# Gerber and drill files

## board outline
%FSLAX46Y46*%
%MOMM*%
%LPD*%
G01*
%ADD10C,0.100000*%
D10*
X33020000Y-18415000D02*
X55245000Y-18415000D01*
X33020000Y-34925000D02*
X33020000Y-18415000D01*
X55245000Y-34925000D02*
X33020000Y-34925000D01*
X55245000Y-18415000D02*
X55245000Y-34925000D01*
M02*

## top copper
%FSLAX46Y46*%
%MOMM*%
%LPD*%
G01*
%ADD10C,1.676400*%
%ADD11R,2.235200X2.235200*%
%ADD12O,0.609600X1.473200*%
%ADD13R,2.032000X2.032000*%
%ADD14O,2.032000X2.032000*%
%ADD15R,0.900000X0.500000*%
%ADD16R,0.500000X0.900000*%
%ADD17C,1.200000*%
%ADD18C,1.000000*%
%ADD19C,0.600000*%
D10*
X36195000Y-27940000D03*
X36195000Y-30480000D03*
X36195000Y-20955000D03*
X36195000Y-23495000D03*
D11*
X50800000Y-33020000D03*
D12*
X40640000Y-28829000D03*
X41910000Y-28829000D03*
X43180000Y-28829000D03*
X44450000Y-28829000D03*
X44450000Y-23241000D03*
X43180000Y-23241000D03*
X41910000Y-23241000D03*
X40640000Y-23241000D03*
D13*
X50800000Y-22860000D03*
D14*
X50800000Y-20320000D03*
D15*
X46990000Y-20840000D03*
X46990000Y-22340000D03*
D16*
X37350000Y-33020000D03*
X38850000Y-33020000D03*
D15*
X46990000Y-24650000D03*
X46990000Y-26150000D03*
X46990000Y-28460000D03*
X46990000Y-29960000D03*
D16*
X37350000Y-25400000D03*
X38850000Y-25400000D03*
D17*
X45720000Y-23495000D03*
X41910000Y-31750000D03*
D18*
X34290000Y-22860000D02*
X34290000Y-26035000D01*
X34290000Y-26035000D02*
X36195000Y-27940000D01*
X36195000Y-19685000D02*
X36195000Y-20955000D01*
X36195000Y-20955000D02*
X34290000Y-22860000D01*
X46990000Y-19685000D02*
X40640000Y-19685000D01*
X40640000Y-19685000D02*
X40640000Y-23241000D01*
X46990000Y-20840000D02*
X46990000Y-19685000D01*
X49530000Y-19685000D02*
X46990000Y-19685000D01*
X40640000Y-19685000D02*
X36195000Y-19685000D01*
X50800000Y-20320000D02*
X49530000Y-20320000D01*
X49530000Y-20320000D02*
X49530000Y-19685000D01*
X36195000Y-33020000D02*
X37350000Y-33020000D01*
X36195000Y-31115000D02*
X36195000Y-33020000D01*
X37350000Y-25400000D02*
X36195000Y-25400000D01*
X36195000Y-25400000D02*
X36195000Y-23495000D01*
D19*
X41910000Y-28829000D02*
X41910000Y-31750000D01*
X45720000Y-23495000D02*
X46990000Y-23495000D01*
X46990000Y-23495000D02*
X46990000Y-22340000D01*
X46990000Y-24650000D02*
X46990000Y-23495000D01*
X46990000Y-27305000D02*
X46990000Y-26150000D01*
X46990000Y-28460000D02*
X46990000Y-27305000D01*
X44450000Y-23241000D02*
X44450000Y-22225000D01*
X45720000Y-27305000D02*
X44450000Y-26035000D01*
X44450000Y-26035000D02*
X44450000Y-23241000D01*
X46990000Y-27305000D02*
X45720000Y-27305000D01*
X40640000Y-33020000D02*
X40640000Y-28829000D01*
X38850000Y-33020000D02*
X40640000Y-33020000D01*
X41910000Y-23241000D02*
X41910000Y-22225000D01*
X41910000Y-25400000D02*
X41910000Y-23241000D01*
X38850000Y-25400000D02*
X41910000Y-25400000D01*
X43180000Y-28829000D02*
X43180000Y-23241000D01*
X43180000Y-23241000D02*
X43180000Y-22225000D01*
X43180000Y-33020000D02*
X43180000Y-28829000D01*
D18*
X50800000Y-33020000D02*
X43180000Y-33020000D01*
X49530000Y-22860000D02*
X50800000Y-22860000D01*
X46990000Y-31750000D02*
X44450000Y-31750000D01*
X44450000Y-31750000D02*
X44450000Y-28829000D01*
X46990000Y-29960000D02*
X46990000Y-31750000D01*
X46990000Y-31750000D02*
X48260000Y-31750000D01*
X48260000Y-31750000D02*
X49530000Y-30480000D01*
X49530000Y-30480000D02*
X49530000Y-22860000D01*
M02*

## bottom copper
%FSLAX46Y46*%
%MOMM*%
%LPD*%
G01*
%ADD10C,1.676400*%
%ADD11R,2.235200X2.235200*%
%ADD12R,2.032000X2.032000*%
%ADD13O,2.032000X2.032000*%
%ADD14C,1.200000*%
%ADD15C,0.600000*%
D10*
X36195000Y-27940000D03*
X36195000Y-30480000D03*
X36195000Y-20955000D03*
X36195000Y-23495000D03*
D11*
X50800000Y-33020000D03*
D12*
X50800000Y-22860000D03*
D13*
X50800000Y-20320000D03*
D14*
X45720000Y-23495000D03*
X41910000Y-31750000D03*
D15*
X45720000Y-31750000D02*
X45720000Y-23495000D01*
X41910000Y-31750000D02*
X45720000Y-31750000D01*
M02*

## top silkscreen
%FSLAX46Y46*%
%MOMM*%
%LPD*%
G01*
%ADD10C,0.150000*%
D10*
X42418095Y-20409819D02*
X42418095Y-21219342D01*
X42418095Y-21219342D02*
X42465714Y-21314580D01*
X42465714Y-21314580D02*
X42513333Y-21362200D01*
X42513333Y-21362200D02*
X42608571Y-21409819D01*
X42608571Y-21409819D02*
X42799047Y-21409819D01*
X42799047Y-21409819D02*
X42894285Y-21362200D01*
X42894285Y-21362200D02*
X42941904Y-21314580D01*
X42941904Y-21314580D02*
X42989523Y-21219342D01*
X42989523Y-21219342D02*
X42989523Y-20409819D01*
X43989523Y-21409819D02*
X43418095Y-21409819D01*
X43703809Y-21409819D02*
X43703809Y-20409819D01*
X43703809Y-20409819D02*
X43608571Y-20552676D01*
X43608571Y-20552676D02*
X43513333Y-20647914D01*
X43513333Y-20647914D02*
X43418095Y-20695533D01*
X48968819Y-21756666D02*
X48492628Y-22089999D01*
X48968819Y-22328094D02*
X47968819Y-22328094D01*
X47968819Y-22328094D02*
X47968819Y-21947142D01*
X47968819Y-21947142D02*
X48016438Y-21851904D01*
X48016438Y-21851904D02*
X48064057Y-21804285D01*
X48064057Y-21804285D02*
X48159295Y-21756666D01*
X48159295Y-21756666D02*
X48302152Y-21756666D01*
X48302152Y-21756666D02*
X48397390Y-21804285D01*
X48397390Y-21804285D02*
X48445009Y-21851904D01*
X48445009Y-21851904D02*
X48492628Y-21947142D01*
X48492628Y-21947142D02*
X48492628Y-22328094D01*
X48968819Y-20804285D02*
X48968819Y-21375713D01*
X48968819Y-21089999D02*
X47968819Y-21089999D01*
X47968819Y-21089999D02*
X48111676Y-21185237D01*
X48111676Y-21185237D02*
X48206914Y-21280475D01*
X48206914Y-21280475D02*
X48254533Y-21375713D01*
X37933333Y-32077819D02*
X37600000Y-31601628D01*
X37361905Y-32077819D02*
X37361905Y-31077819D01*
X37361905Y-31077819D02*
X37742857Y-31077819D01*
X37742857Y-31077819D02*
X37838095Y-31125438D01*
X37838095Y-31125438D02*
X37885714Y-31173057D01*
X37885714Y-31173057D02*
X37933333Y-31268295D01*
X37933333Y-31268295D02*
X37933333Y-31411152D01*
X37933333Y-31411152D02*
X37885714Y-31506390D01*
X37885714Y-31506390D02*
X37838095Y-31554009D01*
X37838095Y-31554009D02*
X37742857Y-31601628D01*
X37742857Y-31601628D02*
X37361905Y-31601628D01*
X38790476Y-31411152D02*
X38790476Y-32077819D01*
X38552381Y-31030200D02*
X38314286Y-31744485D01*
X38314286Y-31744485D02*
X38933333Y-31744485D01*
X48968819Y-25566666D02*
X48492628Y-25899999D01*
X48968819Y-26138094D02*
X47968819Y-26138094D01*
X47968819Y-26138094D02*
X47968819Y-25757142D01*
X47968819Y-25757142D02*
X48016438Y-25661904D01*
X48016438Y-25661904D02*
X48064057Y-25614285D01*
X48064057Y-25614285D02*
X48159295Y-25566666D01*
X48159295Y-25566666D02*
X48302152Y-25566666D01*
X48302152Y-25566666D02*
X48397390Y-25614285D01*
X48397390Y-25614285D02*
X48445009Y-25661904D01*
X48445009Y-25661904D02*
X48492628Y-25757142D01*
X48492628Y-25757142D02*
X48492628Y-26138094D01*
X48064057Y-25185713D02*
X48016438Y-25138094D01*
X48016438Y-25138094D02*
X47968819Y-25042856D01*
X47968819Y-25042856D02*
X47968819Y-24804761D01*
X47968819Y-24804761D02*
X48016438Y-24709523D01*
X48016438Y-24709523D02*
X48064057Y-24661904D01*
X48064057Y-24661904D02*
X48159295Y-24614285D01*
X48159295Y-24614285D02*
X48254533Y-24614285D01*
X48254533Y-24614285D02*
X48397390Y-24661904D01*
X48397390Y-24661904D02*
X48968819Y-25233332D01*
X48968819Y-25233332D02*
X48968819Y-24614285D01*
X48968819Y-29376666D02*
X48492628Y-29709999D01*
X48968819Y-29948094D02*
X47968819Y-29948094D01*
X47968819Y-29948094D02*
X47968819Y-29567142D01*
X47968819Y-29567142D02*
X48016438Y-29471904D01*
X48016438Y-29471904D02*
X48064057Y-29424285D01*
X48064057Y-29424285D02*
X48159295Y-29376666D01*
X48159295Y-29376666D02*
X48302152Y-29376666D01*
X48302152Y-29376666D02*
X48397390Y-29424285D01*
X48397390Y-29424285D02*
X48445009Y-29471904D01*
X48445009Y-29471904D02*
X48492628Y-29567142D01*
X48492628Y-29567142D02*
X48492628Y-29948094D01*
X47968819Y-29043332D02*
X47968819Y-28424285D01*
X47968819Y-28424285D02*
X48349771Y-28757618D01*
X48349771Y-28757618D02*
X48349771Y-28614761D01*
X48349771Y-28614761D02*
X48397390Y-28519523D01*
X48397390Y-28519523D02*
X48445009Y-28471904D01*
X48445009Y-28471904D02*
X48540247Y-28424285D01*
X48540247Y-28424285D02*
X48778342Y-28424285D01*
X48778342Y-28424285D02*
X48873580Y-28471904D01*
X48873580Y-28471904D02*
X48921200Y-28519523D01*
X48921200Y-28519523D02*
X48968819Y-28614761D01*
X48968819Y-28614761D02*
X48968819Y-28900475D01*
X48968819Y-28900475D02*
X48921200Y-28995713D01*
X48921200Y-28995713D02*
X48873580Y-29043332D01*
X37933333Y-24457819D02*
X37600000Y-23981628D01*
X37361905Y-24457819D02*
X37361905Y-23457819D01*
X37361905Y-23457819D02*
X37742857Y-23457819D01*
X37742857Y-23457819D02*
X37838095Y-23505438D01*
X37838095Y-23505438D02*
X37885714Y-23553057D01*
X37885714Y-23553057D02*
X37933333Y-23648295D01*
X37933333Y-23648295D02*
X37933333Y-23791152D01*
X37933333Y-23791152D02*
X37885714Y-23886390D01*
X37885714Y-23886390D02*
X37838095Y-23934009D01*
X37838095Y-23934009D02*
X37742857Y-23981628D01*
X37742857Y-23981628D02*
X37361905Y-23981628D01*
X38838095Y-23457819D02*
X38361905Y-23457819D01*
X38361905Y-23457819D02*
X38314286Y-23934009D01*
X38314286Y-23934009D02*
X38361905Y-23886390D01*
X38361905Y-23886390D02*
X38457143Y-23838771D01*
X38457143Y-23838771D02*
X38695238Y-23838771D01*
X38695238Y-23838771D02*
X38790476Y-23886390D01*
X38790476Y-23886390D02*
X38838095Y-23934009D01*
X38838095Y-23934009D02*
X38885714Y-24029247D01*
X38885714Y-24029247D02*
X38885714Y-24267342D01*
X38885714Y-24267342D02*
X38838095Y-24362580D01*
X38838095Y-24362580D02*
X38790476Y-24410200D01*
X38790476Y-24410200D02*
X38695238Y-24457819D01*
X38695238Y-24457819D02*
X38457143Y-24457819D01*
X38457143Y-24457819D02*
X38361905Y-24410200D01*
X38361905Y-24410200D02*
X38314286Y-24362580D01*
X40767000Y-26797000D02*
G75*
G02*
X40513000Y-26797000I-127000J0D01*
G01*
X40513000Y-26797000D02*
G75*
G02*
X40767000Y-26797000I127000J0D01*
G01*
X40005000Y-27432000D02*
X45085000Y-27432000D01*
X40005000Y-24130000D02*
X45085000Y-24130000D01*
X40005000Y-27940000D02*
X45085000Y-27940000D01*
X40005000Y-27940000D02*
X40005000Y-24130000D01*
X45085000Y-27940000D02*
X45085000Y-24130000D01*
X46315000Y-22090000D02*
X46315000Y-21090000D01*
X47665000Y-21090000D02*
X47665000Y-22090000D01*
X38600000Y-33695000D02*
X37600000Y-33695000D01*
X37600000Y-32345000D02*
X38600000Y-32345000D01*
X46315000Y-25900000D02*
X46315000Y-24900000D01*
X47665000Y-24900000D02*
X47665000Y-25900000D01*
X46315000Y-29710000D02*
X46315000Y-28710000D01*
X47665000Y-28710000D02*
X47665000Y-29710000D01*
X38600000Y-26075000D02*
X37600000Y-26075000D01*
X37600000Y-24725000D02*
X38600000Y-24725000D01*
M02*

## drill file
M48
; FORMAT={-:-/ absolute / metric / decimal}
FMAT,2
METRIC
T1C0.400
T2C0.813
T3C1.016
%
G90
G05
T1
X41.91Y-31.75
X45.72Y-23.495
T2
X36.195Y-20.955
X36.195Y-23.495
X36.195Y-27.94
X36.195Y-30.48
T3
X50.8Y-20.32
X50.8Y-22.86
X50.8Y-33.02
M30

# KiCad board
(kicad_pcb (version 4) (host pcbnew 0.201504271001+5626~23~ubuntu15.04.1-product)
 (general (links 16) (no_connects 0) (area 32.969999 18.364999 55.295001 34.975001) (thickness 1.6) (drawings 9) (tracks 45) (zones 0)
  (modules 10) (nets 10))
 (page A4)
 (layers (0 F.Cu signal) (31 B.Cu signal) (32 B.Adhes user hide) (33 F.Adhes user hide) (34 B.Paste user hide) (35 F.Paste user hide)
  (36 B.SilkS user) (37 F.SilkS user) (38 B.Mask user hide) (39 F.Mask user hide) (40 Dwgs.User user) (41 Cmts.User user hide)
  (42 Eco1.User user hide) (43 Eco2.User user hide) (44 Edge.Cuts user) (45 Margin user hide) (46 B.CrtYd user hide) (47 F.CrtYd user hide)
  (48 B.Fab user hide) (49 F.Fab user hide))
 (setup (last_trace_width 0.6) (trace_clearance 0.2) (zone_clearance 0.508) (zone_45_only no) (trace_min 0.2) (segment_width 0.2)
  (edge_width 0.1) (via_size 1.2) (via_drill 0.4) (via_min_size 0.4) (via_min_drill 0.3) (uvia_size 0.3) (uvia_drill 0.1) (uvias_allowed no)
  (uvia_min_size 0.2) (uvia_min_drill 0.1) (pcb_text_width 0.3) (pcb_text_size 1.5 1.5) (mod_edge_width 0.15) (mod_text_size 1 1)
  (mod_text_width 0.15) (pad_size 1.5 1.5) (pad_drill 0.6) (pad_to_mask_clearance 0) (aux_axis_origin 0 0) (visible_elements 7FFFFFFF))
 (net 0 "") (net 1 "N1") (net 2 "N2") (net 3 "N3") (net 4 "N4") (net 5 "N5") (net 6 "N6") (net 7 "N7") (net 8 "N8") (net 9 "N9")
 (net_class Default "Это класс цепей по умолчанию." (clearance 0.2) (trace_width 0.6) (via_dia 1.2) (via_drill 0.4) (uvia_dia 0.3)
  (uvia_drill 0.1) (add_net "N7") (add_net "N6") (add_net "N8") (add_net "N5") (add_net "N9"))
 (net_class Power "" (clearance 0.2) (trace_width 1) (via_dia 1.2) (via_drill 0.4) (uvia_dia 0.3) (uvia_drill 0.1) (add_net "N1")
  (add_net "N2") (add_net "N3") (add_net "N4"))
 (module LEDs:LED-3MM (layer B.Cu) (at 36.195 29.21 270)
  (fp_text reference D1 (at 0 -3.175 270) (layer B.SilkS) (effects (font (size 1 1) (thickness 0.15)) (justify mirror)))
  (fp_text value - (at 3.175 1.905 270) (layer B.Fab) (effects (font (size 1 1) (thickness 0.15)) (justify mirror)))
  (pad 1 thru_hole circle (at -1.27 0 270) (size 1.6764 1.6764) (drill 0.8128) (layers *.Cu *.Mask B.SilkS) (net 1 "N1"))
  (pad 2 thru_hole circle (at 1.27 0 270) (size 1.6764 1.6764) (drill 0.8128) (layers *.Cu *.Mask B.SilkS) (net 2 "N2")))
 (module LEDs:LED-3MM (layer B.Cu) (at 36.195 22.225 270)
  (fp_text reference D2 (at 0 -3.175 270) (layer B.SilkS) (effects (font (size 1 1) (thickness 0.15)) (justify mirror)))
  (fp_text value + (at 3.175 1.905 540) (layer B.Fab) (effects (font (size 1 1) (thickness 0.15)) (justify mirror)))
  (pad 1 thru_hole circle (at -1.27 0 270) (size 1.6764 1.6764) (drill 0.8128) (layers *.Cu *.Mask B.SilkS) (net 1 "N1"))
  (pad 2 thru_hole circle (at 1.27 0 270) (size 1.6764 1.6764) (drill 0.8128) (layers *.Cu *.Mask B.SilkS) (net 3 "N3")))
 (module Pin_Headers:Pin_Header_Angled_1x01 (layer B.Cu) (at 50.8 33.02)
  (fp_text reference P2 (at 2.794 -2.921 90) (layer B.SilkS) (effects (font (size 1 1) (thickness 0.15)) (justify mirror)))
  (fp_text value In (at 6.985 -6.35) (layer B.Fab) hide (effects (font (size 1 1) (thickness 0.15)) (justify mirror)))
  (pad 1 thru_hole rect (at 0 0) (size 2.2352 2.2352) (drill 1.016) (layers *.Cu *.Mask B.SilkS) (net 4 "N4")))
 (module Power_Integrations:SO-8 (layer F.Cu) (at 42.545 26.035)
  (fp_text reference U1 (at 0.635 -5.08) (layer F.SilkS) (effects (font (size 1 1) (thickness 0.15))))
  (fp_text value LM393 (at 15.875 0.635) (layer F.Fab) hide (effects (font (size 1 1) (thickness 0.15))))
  (fp_circle (center -1.905 0.762) (end -1.778 0.762) (layer F.SilkS) (width 0.15))
  (fp_line (start -2.54 1.397) (end 2.54 1.397) (layer F.SilkS) (width 0.15))
  (fp_line (start -2.54 -1.905) (end 2.54 -1.905) (layer F.SilkS) (width 0.15))
  (fp_line (start -2.54 1.905) (end 2.54 1.905) (layer F.SilkS) (width 0.15))
  (fp_line (start -2.54 1.905) (end -2.54 -1.905) (layer F.SilkS) (width 0.15))
  (fp_line (start 2.54 1.905) (end 2.54 -1.905) (layer F.SilkS) (width 0.15))
  (pad 1 smd oval (at -1.905 2.794) (size 0.6096 1.4732) (layers F.Cu F.Paste F.Mask) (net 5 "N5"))
  (pad 2 smd oval (at -0.635 2.794) (size 0.6096 1.4732) (layers F.Cu F.Paste F.Mask) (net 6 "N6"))
  (pad 3 smd oval (at 0.635 2.794) (size 0.6096 1.4732) (layers F.Cu F.Paste F.Mask) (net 4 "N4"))
  (pad 4 smd oval (at 1.905 2.794) (size 0.6096 1.4732) (layers F.Cu F.Paste F.Mask) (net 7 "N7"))
  (pad 5 smd oval (at 1.905 -2.794) (size 0.6096 1.4732) (layers F.Cu F.Paste F.Mask) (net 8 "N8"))
  (pad 6 smd oval (at 0.635 -2.794) (size 0.6096 1.4732) (layers F.Cu F.Paste F.Mask) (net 4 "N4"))
  (pad 7 smd oval (at -0.635 -2.794) (size 0.6096 1.4732) (layers F.Cu F.Paste F.Mask) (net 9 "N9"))
  (pad 8 smd oval (at -1.905 -2.794) (size 0.6096 1.4732) (layers F.Cu F.Paste F.Mask) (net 1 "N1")))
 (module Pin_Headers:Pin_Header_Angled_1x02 (layer B.Cu) (at 50.8 22.86)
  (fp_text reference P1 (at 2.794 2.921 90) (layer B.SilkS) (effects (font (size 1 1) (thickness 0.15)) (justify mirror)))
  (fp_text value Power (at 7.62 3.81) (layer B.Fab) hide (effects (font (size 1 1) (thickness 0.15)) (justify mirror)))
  (pad 1 thru_hole rect (at 0 0) (size 2.032 2.032) (drill 1.016) (layers *.Cu *.Mask B.SilkS) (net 7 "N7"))
  (pad 2 thru_hole oval (at 0 -2.54) (size 2.032 2.032) (drill 1.016) (layers *.Cu *.Mask B.SilkS) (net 1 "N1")))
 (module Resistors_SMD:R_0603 (layer F.Cu) (at 46.99 21.59 270)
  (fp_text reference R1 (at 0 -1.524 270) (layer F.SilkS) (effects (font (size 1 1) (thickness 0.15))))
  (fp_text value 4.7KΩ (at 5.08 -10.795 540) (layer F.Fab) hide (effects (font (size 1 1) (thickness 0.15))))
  (fp_line (start 0.5 0.675) (end -0.5 0.675) (layer F.SilkS) (width 0.15))
  (fp_line (start -0.5 -0.675) (end 0.5 -0.675) (layer F.SilkS) (width 0.15))
  (pad 1 smd rect (at -0.75 0 270) (size 0.5 0.9) (layers F.Cu F.Paste F.Mask) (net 1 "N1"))
  (pad 2 smd rect (at 0.75 0 270) (size 0.5 0.9) (layers F.Cu F.Paste F.Mask) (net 6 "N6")))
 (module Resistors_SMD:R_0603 (layer F.Cu) (at 38.1 33.02)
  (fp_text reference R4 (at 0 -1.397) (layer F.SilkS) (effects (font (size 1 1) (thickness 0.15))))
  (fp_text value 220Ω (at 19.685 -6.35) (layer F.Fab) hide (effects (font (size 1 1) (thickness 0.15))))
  (fp_line (start 0.5 0.675) (end -0.5 0.675) (layer F.SilkS) (width 0.15))
  (fp_line (start -0.5 -0.675) (end 0.5 -0.675) (layer F.SilkS) (width 0.15))
  (pad 1 smd rect (at -0.75 0) (size 0.5 0.9) (layers F.Cu F.Paste F.Mask) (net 2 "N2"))
  (pad 2 smd rect (at 0.75 0) (size 0.5 0.9) (layers F.Cu F.Paste F.Mask) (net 5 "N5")))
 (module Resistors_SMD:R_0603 (layer F.Cu) (at 46.99 25.4 270)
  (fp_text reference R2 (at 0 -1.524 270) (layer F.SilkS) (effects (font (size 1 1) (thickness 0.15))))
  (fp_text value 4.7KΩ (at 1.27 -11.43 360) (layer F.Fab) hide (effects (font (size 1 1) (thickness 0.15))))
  (fp_line (start 0.5 0.675) (end -0.5 0.675) (layer F.SilkS) (width 0.15))
  (fp_line (start -0.5 -0.675) (end 0.5 -0.675) (layer F.SilkS) (width 0.15))
  (pad 1 smd rect (at -0.75 0 270) (size 0.5 0.9) (layers F.Cu F.Paste F.Mask) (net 6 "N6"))
  (pad 2 smd rect (at 0.75 0 270) (size 0.5 0.9) (layers F.Cu F.Paste F.Mask) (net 8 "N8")))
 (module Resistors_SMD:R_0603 (layer F.Cu) (at 46.99 29.21 270)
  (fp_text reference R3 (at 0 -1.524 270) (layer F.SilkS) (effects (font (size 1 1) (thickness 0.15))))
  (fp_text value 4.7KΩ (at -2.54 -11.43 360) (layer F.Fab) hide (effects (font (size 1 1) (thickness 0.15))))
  (fp_line (start 0.5 0.675) (end -0.5 0.675) (layer F.SilkS) (width 0.15))
  (fp_line (start -0.5 -0.675) (end 0.5 -0.675) (layer F.SilkS) (width 0.15))
  (pad 1 smd rect (at -0.75 0 270) (size 0.5 0.9) (layers F.Cu F.Paste F.Mask) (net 8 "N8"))
  (pad 2 smd rect (at 0.75 0 270) (size 0.5 0.9) (layers F.Cu F.Paste F.Mask) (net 7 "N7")))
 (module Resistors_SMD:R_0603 (layer F.Cu) (at 38.1 25.4)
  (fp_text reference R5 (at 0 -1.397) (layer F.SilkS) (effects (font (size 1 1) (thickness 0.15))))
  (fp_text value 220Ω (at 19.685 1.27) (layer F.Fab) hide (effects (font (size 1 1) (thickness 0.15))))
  (fp_line (start 0.5 0.675) (end -0.5 0.675) (layer F.SilkS) (width 0.15))
  (fp_line (start -0.5 -0.675) (end 0.5 -0.675) (layer F.SilkS) (width 0.15))
  (pad 1 smd rect (at -0.75 0) (size 0.5 0.9) (layers F.Cu F.Paste F.Mask) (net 3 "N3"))
  (pad 2 smd rect (at 0.75 0) (size 0.5 0.9) (layers F.Cu F.Paste F.Mask) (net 9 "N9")))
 (gr_line (start 33.02 18.415) (end 55.245 18.415) (angle 90) (layer Edge.Cuts) (width 0.1))
 (gr_line (start 33.02 34.925) (end 33.02 18.415) (angle 90) (layer Edge.Cuts) (width 0.1))
 (gr_line (start 55.245 34.925) (end 33.02 34.925) (angle 90) (layer Edge.Cuts) (width 0.1))
 (gr_line (start 55.245 18.415) (end 55.245 34.925) (angle 90) (layer Edge.Cuts) (width 0.1))
 (segment (start 34.29 22.86) (end 34.29 26.035) (width 1) (layer F.Cu) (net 1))
 (segment (start 34.29 26.035) (end 36.195 27.94) (width 1) (layer F.Cu) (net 1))
 (segment (start 36.195 19.685) (end 36.195 20.955) (width 1) (layer F.Cu) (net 1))
 (segment (start 36.195 20.955) (end 34.29 22.86) (width 1) (layer F.Cu) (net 1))
 (segment (start 46.99 19.685) (end 40.64 19.685) (width 1) (layer F.Cu) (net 1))
 (segment (start 40.64 19.685) (end 40.64 23.241) (width 1) (layer F.Cu) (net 1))
 (segment (start 46.99 20.84) (end 46.99 19.685) (width 1) (layer F.Cu) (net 1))
 (segment (start 49.53 19.685) (end 46.99 19.685) (width 1) (layer F.Cu) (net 1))
 (segment (start 40.64 19.685) (end 36.195 19.685) (width 1) (layer F.Cu) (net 1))
 (segment (start 50.8 20.32) (end 49.53 20.32) (width 1) (layer F.Cu) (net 1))
 (segment (start 49.53 20.32) (end 49.53 19.685) (width 1) (layer F.Cu) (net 1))
 (segment (start 36.195 33.02) (end 37.35 33.02) (width 1) (layer F.Cu) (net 2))
 (segment (start 36.195 31.115) (end 36.195 33.02) (width 1) (layer F.Cu) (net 2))
 (segment (start 37.35 25.4) (end 36.195 25.4) (width 1) (layer F.Cu) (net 3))
 (segment (start 36.195 25.4) (end 36.195 23.495) (width 1) (layer F.Cu) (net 3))
 (segment (start 41.91 28.829) (end 41.91 31.75) (width 0.6) (layer F.Cu) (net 6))
 (segment (start 45.72 23.495) (end 46.99 23.495) (width 0.6) (layer F.Cu) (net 6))
 (via (at 45.72 23.495) (size 1.2) (layers F.Cu B.Cu) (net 6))
 (segment (start 45.72 31.75) (end 45.72 23.495) (width 0.6) (layer B.Cu) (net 6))
 (segment (start 41.91 31.75) (end 45.72 31.75) (width 0.6) (layer B.Cu) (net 6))
 (via (at 41.91 31.75) (size 1.2) (layers F.Cu B.Cu) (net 6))
 (segment (start 46.99 23.495) (end 46.99 22.34) (width 0.6) (layer F.Cu) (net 6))
 (segment (start 46.99 24.65) (end 46.99 23.495) (width 0.6) (layer F.Cu) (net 6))
 (segment (start 46.99 27.305) (end 46.99 26.15) (width 0.6) (layer F.Cu) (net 8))
 (segment (start 46.99 28.46) (end 46.99 27.305) (width 0.6) (layer F.Cu) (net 8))
 (segment (start 44.45 23.241) (end 44.45 22.225) (width 0.6) (layer F.Cu) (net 8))
 (segment (start 45.72 27.305) (end 44.45 26.035) (width 0.6) (layer F.Cu) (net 8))
 (segment (start 44.45 26.035) (end 44.45 23.241) (width 0.6) (layer F.Cu) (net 8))
 (segment (start 46.99 27.305) (end 45.72 27.305) (width 0.6) (layer F.Cu) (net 8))
 (segment (start 40.64 33.02) (end 40.64 28.829) (width 0.6) (layer F.Cu) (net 5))
 (segment (start 38.85 33.02) (end 40.64 33.02) (width 0.6) (layer F.Cu) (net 5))
 (segment (start 41.91 23.241) (end 41.91 22.225) (width 0.6) (layer F.Cu) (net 9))
 (segment (start 41.91 25.4) (end 41.91 23.241) (width 0.6) (layer F.Cu) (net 9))
 (segment (start 38.85 25.4) (end 41.91 25.4) (width 0.6) (layer F.Cu) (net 9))
 (segment (start 43.18 28.829) (end 43.18 23.241) (width 0.6) (layer F.Cu) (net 4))
 (segment (start 43.18 23.241) (end 43.18 22.225) (width 0.6) (layer F.Cu) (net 4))
 (segment (start 43.18 33.02) (end 43.18 28.829) (width 0.6) (layer F.Cu) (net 4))
 (segment (start 50.8 33.02) (end 43.18 33.02) (width 1) (layer F.Cu) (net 4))
 (segment (start 49.53 22.86) (end 50.8 22.86) (width 1) (layer F.Cu) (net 7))
 (segment (start 46.99 31.75) (end 44.45 31.75) (width 1) (layer F.Cu) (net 7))
 (segment (start 44.45 31.75) (end 44.45 28.829) (width 1) (layer F.Cu) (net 7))
 (segment (start 46.99 29.96) (end 46.99 31.75) (width 1) (layer F.Cu) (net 7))
 (segment (start 46.99 31.75) (end 48.26 31.75) (width 1) (layer F.Cu) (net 7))
 (segment (start 48.26 31.75) (end 49.53 30.48) (width 1) (layer F.Cu) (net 7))
 (segment (start 49.53 30.48) (end 49.53 22.86) (width 1) (layer F.Cu) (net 7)))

